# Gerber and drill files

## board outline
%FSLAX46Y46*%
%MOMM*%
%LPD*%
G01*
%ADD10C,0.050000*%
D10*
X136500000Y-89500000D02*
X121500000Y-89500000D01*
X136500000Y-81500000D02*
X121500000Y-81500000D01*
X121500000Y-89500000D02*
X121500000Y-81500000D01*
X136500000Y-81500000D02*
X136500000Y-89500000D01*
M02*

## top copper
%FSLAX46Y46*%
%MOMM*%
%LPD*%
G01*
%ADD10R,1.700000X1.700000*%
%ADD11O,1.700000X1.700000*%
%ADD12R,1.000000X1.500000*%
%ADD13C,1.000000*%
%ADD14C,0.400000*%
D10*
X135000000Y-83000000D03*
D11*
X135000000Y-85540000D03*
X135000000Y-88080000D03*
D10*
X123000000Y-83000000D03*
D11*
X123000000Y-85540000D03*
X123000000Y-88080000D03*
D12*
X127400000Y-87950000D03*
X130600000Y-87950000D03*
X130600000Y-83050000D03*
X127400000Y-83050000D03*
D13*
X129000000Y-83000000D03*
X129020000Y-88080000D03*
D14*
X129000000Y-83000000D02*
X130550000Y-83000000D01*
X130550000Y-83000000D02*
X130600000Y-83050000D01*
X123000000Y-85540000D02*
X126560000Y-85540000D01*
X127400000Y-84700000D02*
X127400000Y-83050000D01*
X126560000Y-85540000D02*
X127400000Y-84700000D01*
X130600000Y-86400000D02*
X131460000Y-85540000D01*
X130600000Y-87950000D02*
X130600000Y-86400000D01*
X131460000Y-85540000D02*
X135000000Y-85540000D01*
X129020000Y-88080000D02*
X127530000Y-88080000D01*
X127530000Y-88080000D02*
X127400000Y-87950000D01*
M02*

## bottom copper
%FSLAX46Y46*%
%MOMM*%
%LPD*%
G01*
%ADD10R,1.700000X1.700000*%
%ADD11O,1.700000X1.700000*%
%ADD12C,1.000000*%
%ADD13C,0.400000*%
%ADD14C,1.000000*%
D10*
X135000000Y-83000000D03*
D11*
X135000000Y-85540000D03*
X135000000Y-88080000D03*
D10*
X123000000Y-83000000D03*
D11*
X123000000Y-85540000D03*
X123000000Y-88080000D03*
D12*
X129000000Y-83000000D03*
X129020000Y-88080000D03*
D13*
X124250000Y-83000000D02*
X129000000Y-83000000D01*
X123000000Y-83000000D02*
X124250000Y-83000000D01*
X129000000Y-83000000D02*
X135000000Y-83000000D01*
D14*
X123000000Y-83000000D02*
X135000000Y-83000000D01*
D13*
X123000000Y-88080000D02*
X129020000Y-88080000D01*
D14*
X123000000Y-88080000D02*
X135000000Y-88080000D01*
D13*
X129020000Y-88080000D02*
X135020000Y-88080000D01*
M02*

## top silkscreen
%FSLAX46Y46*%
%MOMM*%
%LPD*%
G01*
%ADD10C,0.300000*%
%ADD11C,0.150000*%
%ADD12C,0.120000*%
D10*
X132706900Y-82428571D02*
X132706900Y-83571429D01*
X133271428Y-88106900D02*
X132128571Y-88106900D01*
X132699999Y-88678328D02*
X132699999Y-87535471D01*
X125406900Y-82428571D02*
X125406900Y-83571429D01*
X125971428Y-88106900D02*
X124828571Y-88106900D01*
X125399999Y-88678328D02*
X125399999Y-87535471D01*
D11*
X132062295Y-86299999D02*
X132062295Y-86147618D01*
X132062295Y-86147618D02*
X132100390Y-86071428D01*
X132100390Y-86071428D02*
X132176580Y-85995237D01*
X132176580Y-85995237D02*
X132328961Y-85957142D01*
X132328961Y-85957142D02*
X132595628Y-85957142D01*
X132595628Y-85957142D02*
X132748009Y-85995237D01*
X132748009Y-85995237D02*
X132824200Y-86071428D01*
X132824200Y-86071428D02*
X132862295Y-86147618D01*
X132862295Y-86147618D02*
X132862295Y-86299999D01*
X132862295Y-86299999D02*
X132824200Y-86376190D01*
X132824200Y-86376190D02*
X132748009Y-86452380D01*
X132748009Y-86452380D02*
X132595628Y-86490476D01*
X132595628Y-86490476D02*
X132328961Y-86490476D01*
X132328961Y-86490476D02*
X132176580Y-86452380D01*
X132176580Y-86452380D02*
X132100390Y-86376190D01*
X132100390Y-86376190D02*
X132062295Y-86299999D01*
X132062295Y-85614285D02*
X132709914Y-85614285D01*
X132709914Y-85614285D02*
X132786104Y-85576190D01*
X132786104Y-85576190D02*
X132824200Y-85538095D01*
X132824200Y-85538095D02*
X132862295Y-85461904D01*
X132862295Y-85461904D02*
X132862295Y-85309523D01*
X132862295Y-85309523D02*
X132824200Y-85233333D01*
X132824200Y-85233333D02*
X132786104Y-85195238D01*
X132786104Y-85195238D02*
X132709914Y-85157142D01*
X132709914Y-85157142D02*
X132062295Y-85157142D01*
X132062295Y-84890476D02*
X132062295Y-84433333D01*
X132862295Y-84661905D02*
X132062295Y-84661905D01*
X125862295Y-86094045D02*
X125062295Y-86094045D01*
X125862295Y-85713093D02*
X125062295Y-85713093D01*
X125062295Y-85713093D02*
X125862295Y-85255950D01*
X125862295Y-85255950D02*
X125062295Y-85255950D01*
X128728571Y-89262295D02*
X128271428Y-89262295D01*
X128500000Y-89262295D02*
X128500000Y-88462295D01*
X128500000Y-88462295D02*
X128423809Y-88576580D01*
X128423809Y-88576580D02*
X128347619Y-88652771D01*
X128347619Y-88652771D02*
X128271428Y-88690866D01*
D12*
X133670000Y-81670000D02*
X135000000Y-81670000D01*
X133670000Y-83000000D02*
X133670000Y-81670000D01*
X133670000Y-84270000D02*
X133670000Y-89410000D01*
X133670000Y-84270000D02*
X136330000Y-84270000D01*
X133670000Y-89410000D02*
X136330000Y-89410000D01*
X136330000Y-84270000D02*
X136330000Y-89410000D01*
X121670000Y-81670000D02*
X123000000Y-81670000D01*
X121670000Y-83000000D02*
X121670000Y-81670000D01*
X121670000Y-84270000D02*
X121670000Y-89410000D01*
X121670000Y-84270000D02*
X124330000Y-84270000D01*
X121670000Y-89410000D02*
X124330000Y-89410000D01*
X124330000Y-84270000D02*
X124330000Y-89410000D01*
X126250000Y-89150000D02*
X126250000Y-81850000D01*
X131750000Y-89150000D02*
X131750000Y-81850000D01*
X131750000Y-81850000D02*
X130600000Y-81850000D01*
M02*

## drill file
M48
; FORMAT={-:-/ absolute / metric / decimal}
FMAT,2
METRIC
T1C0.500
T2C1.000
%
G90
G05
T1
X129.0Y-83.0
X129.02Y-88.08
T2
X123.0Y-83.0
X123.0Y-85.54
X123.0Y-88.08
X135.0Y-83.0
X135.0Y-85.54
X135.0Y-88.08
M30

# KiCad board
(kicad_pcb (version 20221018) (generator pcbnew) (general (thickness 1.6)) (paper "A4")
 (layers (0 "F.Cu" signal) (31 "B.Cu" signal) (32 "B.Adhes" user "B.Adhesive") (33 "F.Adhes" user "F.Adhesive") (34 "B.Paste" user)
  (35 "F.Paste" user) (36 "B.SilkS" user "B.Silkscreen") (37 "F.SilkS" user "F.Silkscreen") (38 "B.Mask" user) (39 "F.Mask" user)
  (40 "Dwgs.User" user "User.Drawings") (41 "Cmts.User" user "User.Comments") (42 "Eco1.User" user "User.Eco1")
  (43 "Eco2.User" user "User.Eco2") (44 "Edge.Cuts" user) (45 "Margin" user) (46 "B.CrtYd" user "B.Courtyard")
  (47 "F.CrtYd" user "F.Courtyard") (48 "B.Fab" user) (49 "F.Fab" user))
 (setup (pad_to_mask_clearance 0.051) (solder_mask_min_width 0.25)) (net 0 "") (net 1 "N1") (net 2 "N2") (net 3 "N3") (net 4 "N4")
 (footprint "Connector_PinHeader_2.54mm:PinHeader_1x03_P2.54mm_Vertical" (layer "F.Cu") (at 135 83)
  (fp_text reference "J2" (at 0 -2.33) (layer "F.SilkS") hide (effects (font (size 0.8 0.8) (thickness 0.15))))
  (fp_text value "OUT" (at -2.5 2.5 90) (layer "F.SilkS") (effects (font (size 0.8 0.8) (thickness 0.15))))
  (fp_line (start -1.33 -1.33) (end 0 -1.33) (stroke (width 0.12) (type solid)) (layer "F.SilkS"))
  (fp_line (start -1.33 0) (end -1.33 -1.33) (stroke (width 0.12) (type solid)) (layer "F.SilkS"))
  (fp_line (start -1.33 1.27) (end -1.33 6.41) (stroke (width 0.12) (type solid)) (layer "F.SilkS"))
  (fp_line (start -1.33 1.27) (end 1.33 1.27) (stroke (width 0.12) (type solid)) (layer "F.SilkS"))
  (fp_line (start -1.33 6.41) (end 1.33 6.41) (stroke (width 0.12) (type solid)) (layer "F.SilkS"))
  (fp_line (start 1.33 1.27) (end 1.33 6.41) (stroke (width 0.12) (type solid)) (layer "F.SilkS"))
  (pad "1" thru_hole rect (at 0 0) (size 1.7 1.7) (drill 1) (layers "*.Cu" "*.Mask") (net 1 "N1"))
  (pad "2" thru_hole oval (at 0 2.54) (size 1.7 1.7) (drill 1) (layers "*.Cu" "*.Mask") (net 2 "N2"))
  (pad "3" thru_hole oval (at 0 5.08) (size 1.7 1.7) (drill 1) (layers "*.Cu" "*.Mask") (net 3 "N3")))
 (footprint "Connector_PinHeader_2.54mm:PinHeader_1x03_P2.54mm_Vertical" (layer "F.Cu") (at 123 83)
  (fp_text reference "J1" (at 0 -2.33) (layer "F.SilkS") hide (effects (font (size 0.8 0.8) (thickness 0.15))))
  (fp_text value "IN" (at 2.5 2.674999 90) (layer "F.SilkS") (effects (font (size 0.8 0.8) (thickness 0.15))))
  (fp_line (start -1.33 -1.33) (end 0 -1.33) (stroke (width 0.12) (type solid)) (layer "F.SilkS"))
  (fp_line (start -1.33 0) (end -1.33 -1.33) (stroke (width 0.12) (type solid)) (layer "F.SilkS"))
  (fp_line (start -1.33 1.27) (end -1.33 6.41) (stroke (width 0.12) (type solid)) (layer "F.SilkS"))
  (fp_line (start -1.33 1.27) (end 1.33 1.27) (stroke (width 0.12) (type solid)) (layer "F.SilkS"))
  (fp_line (start -1.33 6.41) (end 1.33 6.41) (stroke (width 0.12) (type solid)) (layer "F.SilkS"))
  (fp_line (start 1.33 1.27) (end 1.33 6.41) (stroke (width 0.12) (type solid)) (layer "F.SilkS"))
  (pad "1" thru_hole rect (at 0 0) (size 1.7 1.7) (drill 1) (layers "*.Cu" "*.Mask") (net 1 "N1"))
  (pad "2" thru_hole oval (at 0 2.54) (size 1.7 1.7) (drill 1) (layers "*.Cu" "*.Mask") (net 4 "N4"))
  (pad "3" thru_hole oval (at 0 5.08) (size 1.7 1.7) (drill 1) (layers "*.Cu" "*.Mask") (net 3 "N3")))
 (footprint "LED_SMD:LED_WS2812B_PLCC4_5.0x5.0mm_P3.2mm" (layer "F.Cu") (at 129 85.5 90)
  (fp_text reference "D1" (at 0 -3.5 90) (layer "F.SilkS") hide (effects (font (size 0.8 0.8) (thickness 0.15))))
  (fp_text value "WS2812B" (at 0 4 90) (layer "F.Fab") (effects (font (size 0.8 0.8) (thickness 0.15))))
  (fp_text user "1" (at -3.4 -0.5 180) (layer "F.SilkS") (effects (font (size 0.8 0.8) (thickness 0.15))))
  (fp_line (start -3.65 -2.75) (end 3.65 -2.75) (stroke (width 0.12) (type solid)) (layer "F.SilkS"))
  (fp_line (start -3.65 2.75) (end 3.65 2.75) (stroke (width 0.12) (type solid)) (layer "F.SilkS"))
  (fp_line (start 3.65 2.75) (end 3.65 1.6) (stroke (width 0.12) (type solid)) (layer "F.SilkS"))
  (pad "1" smd rect (at -2.45 -1.6 90) (size 1.5 1) (layers "F.Cu" "F.Paste" "F.Mask") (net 3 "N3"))
  (pad "2" smd rect (at -2.45 1.6 90) (size 1.5 1) (layers "F.Cu" "F.Paste" "F.Mask") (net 2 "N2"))
  (pad "3" smd rect (at 2.45 1.6 90) (size 1.5 1) (layers "F.Cu" "F.Paste" "F.Mask") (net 1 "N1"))
  (pad "4" smd rect (at 2.45 -1.6 90) (size 1.5 1) (layers "F.Cu" "F.Paste" "F.Mask") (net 4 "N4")))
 (gr_line (start 136.5 89.5) (end 121.5 89.5) (stroke (width 0.05) (type solid)) (layer "Edge.Cuts"))
 (gr_line (start 136.5 81.5) (end 121.5 81.5) (stroke (width 0.05) (type solid)) (layer "Edge.Cuts"))
 (gr_line (start 121.5 89.5) (end 121.5 81.5) (stroke (width 0.05) (type solid)) (layer "Edge.Cuts"))
 (gr_line (start 136.5 81.5) (end 136.5 89.5) (stroke (width 0.05) (type solid)) (layer "Edge.Cuts"))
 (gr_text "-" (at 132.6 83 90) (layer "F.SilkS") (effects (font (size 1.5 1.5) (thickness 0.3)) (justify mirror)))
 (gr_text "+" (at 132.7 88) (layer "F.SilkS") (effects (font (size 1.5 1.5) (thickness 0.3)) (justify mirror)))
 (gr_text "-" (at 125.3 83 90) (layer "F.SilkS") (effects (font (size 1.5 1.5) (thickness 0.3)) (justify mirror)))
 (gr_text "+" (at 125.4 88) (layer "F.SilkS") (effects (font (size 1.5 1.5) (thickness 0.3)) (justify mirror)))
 (segment (start 129 83) (end 130.55 83) (width 0.4) (layer "F.Cu") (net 1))
 (segment (start 130.55 83) (end 130.6 83.05) (width 0.4) (layer "F.Cu") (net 1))
 (via (at 129 83) (size 1) (drill 0.5) (layers "F.Cu" "B.Cu") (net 1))
 (segment (start 124.25 83) (end 129 83) (width 0.4) (layer "B.Cu") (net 1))
 (segment (start 123 83) (end 124.25 83) (width 0.4) (layer "B.Cu") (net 1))
 (segment (start 129 83) (end 135 83) (width 0.4) (layer "B.Cu") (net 1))
 (segment (start 123 83) (end 135 83) (width 1) (layer "B.Cu") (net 1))
 (segment (start 123 85.54) (end 126.56 85.54) (width 0.4) (layer "F.Cu") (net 4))
 (segment (start 127.4 84.7) (end 127.4 83.05) (width 0.4) (layer "F.Cu") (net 4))
 (segment (start 126.56 85.54) (end 127.4 84.7) (width 0.4) (layer "F.Cu") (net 4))
 (segment (start 130.6 86.4) (end 131.46 85.54) (width 0.4) (layer "F.Cu") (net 2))
 (segment (start 130.6 87.95) (end 130.6 86.4) (width 0.4) (layer "F.Cu") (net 2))
 (segment (start 131.46 85.54) (end 135 85.54) (width 0.4) (layer "F.Cu") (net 2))
 (segment (start 129.02 88.08) (end 127.53 88.08) (width 0.4) (layer "F.Cu") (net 3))
 (segment (start 127.53 88.08) (end 127.4 87.95) (width 0.4) (layer "F.Cu") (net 3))
 (via (at 129.02 88.08) (size 1) (drill 0.5) (layers "F.Cu" "B.Cu") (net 3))
 (segment (start 123 88.08) (end 129.02 88.08) (width 0.4) (layer "B.Cu") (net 3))
 (segment (start 123 88.08) (end 135 88.08) (width 1) (layer "B.Cu") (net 3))
 (segment (start 129.02 88.08) (end 135.02 88.08) (width 0.4) (layer "B.Cu") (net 3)))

